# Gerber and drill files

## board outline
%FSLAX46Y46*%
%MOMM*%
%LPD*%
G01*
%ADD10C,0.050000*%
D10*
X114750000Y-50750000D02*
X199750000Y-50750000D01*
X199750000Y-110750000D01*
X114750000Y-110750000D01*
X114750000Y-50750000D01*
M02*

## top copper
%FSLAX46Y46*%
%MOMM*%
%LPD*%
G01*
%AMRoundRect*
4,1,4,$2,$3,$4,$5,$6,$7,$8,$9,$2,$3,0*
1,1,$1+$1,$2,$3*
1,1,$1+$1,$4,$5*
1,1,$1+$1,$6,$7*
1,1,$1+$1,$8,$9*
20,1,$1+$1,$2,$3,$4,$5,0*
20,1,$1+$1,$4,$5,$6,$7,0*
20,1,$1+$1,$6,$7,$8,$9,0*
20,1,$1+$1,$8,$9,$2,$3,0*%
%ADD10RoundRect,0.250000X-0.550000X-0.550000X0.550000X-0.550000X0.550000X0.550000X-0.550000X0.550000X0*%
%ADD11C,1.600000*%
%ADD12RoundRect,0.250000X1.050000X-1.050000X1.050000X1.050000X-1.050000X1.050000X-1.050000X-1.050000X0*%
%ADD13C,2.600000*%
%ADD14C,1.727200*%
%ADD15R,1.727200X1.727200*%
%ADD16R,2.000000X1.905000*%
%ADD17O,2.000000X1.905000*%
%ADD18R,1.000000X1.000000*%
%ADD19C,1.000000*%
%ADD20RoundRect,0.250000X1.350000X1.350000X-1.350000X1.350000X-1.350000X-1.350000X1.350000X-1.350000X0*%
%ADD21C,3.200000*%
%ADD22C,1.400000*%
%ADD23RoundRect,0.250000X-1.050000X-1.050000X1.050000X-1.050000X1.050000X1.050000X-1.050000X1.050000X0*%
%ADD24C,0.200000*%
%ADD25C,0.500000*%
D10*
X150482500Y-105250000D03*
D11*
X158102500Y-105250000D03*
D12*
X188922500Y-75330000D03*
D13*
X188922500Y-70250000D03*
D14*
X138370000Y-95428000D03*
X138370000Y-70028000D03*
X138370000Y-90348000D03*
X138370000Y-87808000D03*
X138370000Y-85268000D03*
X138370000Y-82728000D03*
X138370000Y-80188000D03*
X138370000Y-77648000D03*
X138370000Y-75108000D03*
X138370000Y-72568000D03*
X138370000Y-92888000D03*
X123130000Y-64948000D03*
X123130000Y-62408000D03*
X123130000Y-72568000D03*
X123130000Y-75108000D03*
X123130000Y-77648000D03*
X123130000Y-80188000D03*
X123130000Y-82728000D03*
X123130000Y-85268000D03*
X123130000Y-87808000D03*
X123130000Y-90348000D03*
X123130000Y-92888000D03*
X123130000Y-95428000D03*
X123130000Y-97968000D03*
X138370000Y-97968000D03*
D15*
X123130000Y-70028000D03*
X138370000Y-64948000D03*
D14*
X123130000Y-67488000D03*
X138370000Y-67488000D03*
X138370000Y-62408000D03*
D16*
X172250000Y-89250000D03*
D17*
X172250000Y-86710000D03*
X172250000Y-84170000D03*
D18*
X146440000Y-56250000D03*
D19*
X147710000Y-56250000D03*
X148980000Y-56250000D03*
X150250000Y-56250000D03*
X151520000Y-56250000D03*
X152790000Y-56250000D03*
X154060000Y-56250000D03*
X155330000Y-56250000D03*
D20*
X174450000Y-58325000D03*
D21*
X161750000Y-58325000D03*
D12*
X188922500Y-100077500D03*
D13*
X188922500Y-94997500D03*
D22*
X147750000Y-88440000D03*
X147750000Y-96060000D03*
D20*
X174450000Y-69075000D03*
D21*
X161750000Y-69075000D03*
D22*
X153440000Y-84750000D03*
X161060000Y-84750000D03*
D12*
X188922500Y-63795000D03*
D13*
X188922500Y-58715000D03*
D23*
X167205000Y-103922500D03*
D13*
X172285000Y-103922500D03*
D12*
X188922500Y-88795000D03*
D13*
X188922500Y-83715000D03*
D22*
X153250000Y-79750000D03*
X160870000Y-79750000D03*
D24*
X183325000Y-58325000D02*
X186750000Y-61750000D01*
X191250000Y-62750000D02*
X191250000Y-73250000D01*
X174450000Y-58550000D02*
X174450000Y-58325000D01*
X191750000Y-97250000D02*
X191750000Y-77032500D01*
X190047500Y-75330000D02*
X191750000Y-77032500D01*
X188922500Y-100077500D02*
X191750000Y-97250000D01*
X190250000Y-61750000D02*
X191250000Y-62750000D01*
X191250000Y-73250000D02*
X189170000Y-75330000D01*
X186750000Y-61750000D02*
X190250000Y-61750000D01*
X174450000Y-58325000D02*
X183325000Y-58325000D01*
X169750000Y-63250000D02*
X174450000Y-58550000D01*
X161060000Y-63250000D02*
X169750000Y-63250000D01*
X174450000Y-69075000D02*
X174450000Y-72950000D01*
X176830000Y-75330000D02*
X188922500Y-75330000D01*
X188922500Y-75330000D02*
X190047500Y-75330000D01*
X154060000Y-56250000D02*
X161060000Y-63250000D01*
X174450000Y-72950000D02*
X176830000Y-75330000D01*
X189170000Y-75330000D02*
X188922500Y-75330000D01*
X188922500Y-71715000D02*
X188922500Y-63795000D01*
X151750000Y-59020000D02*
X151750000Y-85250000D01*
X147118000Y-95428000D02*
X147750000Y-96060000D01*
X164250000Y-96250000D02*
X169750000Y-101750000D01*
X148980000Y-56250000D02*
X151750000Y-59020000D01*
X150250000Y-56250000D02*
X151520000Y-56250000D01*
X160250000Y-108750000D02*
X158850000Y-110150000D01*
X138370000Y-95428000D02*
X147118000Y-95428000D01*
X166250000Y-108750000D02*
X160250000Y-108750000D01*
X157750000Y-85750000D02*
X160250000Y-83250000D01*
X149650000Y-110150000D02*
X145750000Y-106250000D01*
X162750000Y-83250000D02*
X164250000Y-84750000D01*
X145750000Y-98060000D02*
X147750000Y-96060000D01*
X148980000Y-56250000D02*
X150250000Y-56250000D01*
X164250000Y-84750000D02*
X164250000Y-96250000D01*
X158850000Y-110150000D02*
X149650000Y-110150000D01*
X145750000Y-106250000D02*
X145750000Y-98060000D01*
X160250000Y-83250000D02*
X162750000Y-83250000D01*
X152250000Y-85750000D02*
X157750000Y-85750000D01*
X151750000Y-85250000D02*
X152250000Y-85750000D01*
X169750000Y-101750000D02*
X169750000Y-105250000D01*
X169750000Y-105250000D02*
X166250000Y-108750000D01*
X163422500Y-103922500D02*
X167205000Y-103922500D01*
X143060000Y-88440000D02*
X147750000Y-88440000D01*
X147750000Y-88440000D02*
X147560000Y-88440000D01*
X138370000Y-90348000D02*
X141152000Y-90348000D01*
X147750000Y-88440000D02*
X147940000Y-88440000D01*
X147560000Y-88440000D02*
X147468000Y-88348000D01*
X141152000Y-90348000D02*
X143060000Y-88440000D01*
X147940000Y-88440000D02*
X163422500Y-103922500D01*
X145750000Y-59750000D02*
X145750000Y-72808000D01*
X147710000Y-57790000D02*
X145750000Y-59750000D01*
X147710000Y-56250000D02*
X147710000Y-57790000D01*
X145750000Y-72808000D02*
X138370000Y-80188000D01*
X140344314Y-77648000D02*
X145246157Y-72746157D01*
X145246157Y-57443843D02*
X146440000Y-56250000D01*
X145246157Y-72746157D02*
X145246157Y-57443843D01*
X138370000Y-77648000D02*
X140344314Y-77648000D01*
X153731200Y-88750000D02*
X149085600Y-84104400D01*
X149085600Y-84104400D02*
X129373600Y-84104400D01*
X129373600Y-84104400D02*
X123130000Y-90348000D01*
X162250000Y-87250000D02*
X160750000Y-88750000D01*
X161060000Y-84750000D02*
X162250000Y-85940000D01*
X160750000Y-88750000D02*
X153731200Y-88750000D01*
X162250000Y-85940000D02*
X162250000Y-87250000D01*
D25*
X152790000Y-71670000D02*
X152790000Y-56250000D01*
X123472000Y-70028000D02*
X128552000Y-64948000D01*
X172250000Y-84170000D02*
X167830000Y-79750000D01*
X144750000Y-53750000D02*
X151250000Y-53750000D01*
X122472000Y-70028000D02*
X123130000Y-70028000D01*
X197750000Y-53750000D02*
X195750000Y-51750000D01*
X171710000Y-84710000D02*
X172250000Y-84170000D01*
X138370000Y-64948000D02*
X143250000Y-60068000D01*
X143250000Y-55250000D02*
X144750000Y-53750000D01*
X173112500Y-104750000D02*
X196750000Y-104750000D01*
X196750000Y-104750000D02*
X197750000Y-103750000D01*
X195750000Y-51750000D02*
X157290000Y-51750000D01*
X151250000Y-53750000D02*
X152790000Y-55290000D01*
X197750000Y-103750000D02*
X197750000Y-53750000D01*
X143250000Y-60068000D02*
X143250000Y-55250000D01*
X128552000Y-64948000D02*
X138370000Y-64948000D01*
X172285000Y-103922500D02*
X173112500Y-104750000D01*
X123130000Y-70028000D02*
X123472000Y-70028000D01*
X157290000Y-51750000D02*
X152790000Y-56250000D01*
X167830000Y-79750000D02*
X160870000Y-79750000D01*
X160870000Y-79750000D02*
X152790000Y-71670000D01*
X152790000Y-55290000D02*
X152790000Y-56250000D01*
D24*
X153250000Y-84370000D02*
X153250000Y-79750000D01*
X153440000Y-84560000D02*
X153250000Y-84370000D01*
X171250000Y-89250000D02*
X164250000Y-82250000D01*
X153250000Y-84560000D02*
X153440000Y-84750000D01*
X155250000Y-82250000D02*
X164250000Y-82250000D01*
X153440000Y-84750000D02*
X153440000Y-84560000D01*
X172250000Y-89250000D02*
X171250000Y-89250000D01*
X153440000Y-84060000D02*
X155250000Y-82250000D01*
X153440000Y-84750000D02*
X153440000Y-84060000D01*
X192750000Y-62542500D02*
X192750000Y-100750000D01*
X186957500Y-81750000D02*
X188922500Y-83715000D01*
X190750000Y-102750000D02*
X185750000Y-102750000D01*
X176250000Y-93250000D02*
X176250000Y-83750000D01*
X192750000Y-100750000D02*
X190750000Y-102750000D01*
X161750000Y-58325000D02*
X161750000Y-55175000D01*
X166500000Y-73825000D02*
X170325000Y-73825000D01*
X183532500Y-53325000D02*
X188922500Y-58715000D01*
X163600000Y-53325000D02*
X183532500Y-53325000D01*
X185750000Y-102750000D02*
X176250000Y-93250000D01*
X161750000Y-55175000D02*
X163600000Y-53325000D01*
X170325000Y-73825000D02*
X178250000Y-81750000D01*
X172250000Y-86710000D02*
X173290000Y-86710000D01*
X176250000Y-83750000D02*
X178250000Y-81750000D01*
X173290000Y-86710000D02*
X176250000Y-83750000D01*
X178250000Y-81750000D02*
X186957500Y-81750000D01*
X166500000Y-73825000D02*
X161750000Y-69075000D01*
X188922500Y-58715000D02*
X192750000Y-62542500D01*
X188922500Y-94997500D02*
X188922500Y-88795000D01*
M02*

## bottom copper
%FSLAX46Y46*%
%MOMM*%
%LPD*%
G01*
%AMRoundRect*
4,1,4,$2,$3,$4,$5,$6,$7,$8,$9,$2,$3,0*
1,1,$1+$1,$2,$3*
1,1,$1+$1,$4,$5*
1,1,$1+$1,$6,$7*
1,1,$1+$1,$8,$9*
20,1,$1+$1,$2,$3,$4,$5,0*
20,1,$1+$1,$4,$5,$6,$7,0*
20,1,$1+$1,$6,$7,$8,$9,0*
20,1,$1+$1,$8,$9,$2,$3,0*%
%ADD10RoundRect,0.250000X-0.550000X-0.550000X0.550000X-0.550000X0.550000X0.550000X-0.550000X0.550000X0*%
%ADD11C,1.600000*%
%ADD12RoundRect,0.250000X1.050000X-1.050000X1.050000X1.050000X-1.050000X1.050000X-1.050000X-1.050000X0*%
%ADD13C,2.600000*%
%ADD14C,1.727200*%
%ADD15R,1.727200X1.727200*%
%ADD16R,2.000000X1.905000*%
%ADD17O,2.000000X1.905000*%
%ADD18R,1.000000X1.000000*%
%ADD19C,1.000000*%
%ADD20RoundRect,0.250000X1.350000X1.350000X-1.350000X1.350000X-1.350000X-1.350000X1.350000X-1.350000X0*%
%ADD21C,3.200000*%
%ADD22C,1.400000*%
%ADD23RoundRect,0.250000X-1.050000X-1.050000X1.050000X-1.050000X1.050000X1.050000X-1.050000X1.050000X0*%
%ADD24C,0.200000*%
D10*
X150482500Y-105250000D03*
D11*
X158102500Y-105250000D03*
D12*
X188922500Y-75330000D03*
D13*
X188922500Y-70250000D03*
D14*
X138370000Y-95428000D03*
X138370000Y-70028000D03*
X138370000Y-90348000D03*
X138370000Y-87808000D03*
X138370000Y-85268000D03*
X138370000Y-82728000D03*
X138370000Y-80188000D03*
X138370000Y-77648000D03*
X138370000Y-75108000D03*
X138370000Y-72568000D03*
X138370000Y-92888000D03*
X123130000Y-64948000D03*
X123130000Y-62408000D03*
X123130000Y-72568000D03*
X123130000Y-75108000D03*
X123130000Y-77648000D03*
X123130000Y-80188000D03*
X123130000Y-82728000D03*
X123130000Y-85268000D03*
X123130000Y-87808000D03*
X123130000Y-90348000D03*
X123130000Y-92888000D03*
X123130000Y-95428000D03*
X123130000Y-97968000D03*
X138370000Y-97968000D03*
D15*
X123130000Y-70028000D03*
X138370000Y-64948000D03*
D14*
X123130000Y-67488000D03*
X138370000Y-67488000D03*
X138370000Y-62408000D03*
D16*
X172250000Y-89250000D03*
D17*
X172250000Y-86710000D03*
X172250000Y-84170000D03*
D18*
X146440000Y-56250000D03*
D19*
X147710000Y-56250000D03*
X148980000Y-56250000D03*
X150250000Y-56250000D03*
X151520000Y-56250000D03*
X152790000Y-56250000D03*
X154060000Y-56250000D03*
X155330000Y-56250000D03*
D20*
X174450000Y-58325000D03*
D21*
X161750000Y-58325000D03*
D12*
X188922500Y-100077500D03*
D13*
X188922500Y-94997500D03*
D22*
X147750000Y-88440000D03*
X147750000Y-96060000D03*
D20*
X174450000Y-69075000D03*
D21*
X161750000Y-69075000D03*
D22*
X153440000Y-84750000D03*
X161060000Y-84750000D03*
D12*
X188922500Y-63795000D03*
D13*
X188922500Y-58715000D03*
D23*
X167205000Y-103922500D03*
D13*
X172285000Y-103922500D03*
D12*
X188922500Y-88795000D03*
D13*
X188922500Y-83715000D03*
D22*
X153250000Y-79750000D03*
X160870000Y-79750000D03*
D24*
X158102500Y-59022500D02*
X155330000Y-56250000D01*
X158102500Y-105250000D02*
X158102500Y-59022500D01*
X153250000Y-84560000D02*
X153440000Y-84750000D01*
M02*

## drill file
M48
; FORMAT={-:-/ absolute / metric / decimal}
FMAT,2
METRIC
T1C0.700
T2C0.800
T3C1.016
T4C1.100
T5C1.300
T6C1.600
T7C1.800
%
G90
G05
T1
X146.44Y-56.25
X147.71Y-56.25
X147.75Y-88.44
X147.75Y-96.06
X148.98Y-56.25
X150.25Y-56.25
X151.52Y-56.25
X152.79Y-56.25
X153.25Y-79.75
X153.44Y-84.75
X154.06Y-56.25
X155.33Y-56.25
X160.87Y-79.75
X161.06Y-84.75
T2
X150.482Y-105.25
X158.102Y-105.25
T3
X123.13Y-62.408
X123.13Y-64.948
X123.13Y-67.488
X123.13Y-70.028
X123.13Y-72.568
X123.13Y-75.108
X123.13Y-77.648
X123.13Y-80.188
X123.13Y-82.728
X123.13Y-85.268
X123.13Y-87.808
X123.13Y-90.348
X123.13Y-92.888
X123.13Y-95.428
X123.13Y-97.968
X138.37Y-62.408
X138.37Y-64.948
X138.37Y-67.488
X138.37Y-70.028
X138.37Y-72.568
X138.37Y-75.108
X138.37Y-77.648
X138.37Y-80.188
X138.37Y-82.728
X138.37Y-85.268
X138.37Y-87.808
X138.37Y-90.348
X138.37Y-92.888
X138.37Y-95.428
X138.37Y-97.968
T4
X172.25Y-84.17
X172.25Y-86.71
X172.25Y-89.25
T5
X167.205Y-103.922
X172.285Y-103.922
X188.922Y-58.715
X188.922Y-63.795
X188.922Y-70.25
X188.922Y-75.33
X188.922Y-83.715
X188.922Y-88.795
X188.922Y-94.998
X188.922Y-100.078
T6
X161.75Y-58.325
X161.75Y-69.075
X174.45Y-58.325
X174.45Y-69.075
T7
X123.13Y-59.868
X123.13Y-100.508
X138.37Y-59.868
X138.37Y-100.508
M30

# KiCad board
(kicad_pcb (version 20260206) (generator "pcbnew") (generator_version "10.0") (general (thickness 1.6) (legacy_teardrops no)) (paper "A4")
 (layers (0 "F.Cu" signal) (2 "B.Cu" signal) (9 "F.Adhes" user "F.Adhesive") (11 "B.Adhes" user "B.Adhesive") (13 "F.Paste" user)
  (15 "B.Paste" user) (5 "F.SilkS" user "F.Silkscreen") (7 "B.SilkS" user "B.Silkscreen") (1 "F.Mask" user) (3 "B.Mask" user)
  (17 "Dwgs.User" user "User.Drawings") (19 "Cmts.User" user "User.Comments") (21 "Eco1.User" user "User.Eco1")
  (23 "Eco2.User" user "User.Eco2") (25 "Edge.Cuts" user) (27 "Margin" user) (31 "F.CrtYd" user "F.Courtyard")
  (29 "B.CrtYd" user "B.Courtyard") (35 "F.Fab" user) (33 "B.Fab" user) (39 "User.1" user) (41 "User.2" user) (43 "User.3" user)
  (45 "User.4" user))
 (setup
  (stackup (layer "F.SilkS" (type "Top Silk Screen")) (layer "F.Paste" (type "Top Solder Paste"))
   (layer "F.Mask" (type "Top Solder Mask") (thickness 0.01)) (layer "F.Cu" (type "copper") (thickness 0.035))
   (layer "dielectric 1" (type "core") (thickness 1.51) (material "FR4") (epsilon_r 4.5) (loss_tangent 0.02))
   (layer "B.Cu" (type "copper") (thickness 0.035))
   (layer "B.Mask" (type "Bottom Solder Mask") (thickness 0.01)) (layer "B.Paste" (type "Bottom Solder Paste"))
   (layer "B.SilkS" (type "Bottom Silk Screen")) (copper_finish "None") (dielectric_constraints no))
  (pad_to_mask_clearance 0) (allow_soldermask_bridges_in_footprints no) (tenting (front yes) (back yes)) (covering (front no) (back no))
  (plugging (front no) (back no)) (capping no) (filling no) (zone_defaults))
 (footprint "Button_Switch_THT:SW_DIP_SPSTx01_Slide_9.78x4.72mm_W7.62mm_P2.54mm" (layer "F.Cu") (at 150.4825 105.25)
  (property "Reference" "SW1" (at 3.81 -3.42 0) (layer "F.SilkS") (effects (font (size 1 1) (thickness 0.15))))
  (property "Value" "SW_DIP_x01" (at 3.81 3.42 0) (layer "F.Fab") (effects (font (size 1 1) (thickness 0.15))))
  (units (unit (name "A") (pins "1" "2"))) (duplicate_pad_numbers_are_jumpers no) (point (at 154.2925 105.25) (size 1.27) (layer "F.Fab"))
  (pad "1" thru_hole roundrect (at 0 0) (size 1.6 1.6) (drill 0.8) (layers "*.Cu" "*.Mask") (remove_unused_layers no)
   (roundrect_rratio 0.15625) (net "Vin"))
  (pad "2" thru_hole circle (at 7.62 0) (size 1.6 1.6) (drill 0.8) (layers "*.Cu" "*.Mask") (remove_unused_layers no) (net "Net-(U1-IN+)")))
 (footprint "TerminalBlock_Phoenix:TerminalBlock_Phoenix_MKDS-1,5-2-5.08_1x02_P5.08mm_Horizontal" (layer "F.Cu") (at 188.9225 75.33 90)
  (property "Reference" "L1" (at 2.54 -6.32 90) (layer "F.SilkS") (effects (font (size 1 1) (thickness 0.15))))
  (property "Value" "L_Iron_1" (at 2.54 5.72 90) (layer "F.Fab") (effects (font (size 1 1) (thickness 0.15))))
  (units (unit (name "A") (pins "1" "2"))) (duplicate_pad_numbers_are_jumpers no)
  (pad "1" thru_hole roundrect (at 0 0 90) (size 2.6 2.6) (drill 1.3) (layers "*.Cu" "*.Mask") (remove_unused_layers no)
   (roundrect_rratio 0.096154) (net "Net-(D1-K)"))
  (pad "2" thru_hole circle (at 5.08 0 90) (size 2.6 2.6) (drill 1.3) (layers "*.Cu" "*.Mask") (remove_unused_layers no)
   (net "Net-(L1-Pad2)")))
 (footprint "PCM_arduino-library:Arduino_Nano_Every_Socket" (layer "F.Cu") (at 130.75 101.778)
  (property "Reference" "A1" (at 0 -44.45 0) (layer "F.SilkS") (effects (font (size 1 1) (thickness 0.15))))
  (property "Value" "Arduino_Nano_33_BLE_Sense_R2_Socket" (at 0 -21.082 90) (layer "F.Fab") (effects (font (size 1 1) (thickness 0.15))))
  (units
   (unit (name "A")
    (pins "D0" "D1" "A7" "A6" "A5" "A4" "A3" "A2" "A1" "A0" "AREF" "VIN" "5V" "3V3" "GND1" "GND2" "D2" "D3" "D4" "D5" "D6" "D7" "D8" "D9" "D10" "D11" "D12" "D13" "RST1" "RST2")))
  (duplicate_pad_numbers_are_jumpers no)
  (pad "" np_thru_hole circle (at -7.62 -41.91) (size 1.8 1.8) (drill 1.8) (layers "*.Cu" "*.Mask"))
  (pad "" np_thru_hole circle (at -7.62 -1.27) (size 1.8 1.8) (drill 1.8) (layers "*.Cu" "*.Mask"))
  (pad "" np_thru_hole circle (at 7.62 -41.91) (size 1.8 1.8) (drill 1.8) (layers "*.Cu" "*.Mask"))
  (pad "" np_thru_hole circle (at 7.62 -1.27) (size 1.8 1.8) (drill 1.8) (layers "*.Cu" "*.Mask"))
  (pad "3V3" thru_hole circle (at 7.62 -6.35) (size 1.7272 1.7272) (drill 1.016) (layers "*.Cu" "*.Mask") (remove_unused_layers no)
   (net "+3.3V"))
  (pad "5V" thru_hole circle (at 7.62 -31.75) (size 1.7272 1.7272) (drill 1.016) (layers "*.Cu" "*.Mask") (remove_unused_layers no)
   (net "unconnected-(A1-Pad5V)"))
  (pad "A0" thru_hole circle (at 7.62 -11.43) (size 1.7272 1.7272) (drill 1.016) (layers "*.Cu" "*.Mask") (remove_unused_layers no)
   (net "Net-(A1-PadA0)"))
  (pad "A1" thru_hole circle (at 7.62 -13.97) (size 1.7272 1.7272) (drill 1.016) (layers "*.Cu" "*.Mask") (remove_unused_layers no)
   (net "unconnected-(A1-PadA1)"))
  (pad "A2" thru_hole circle (at 7.62 -16.51) (size 1.7272 1.7272) (drill 1.016) (layers "*.Cu" "*.Mask") (remove_unused_layers no)
   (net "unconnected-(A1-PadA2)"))
  (pad "A3" thru_hole circle (at 7.62 -19.05) (size 1.7272 1.7272) (drill 1.016) (layers "*.Cu" "*.Mask") (remove_unused_layers no)
   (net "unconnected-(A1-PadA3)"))
  (pad "A4" thru_hole circle (at 7.62 -21.59) (size 1.7272 1.7272) (drill 1.016) (layers "*.Cu" "*.Mask") (remove_unused_layers no)
   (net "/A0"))
  (pad "A5" thru_hole circle (at 7.62 -24.13) (size 1.7272 1.7272) (drill 1.016) (layers "*.Cu" "*.Mask") (remove_unused_layers no)
   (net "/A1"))
  (pad "A6" thru_hole circle (at 7.62 -26.67) (size 1.7272 1.7272) (drill 1.016) (layers "*.Cu" "*.Mask") (remove_unused_layers no)
   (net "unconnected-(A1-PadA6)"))
  (pad "A7" thru_hole circle (at 7.62 -29.21) (size 1.7272 1.7272) (drill 1.016) (layers "*.Cu" "*.Mask") (remove_unused_layers no)
   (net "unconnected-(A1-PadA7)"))
  (pad "AREF" thru_hole circle (at 7.62 -8.89) (size 1.7272 1.7272) (drill 1.016) (layers "*.Cu" "*.Mask") (remove_unused_layers no)
   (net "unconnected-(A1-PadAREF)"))
  (pad "D0" thru_hole circle (at -7.62 -36.83) (size 1.7272 1.7272) (drill 1.016) (layers "*.Cu" "*.Mask") (remove_unused_layers no)
   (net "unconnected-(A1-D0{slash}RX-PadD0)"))
  (pad "D1" thru_hole circle (at -7.62 -39.37) (size 1.7272 1.7272) (drill 1.016) (layers "*.Cu" "*.Mask") (remove_unused_layers no)
   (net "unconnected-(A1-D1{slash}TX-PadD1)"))
  (pad "D2" thru_hole circle (at -7.62 -29.21) (size 1.7272 1.7272) (drill 1.016) (layers "*.Cu" "*.Mask") (remove_unused_layers no)
   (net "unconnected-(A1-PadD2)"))
  (pad "D3" thru_hole circle (at -7.62 -26.67) (size 1.7272 1.7272) (drill 1.016) (layers "*.Cu" "*.Mask") (remove_unused_layers no)
   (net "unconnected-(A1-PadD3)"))
  (pad "D4" thru_hole circle (at -7.62 -24.13) (size 1.7272 1.7272) (drill 1.016) (layers "*.Cu" "*.Mask") (remove_unused_layers no)
   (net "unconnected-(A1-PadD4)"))
  (pad "D5" thru_hole circle (at -7.62 -21.59) (size 1.7272 1.7272) (drill 1.016) (layers "*.Cu" "*.Mask") (remove_unused_layers no)
   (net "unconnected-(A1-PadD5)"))
  (pad "D6" thru_hole circle (at -7.62 -19.05) (size 1.7272 1.7272) (drill 1.016) (layers "*.Cu" "*.Mask") (remove_unused_layers no)
   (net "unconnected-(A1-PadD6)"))
  (pad "D7" thru_hole circle (at -7.62 -16.51) (size 1.7272 1.7272) (drill 1.016) (layers "*.Cu" "*.Mask") (remove_unused_layers no)
   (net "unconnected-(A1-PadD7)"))
  (pad "D8" thru_hole circle (at -7.62 -13.97) (size 1.7272 1.7272) (drill 1.016) (layers "*.Cu" "*.Mask") (remove_unused_layers no)
   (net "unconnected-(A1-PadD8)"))
  (pad "D9" thru_hole circle (at -7.62 -11.43) (size 1.7272 1.7272) (drill 1.016) (layers "*.Cu" "*.Mask") (remove_unused_layers no)
   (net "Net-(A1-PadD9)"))
  (pad "D10" thru_hole circle (at -7.62 -8.89) (size 1.7272 1.7272) (drill 1.016) (layers "*.Cu" "*.Mask") (remove_unused_layers no)
   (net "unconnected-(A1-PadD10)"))
  (pad "D11" thru_hole circle (at -7.62 -6.35) (size 1.7272 1.7272) (drill 1.016) (layers "*.Cu" "*.Mask") (remove_unused_layers no)
   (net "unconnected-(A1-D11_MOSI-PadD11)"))
  (pad "D12" thru_hole circle (at -7.62 -3.81) (size 1.7272 1.7272) (drill 1.016) (layers "*.Cu" "*.Mask") (remove_unused_layers no)
   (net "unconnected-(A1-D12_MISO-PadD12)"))
  (pad "D13" thru_hole circle (at 7.62 -3.81) (size 1.7272 1.7272) (drill 1.016) (layers "*.Cu" "*.Mask") (remove_unused_layers no)
   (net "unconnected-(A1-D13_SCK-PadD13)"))
  (pad "GND1" thru_hole rect (at -7.62 -31.75) (size 1.7272 1.7272) (drill 1.016) (layers "*.Cu" "*.Mask") (remove_unused_layers no)
   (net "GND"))
  (pad "GND2" thru_hole rect (at 7.62 -36.83) (size 1.7272 1.7272) (drill 1.016) (layers "*.Cu" "*.Mask") (remove_unused_layers no)
   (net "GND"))
  (pad "RST1" thru_hole circle (at -7.62 -34.29) (size 1.7272 1.7272) (drill 1.016) (layers "*.Cu" "*.Mask") (remove_unused_layers no)
   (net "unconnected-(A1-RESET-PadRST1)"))
  (pad "RST2" thru_hole circle (at 7.62 -34.29) (size 1.7272 1.7272) (drill 1.016) (layers "*.Cu" "*.Mask") (remove_unused_layers no)
   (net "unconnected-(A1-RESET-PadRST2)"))
  (pad "VIN" thru_hole circle (at 7.62 -39.37) (size 1.7272 1.7272) (drill 1.016) (layers "*.Cu" "*.Mask") (remove_unused_layers no)
   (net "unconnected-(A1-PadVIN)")))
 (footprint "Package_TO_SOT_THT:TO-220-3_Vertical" (layer "F.Cu") (at 172.25 89.25 90)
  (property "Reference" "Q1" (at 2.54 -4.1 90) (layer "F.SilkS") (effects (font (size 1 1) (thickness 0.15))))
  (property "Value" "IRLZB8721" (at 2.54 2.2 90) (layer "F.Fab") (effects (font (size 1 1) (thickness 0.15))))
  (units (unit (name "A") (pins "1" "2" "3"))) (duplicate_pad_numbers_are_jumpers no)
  (pad "1" thru_hole rect (at 0 0 90) (size 1.905 2) (drill 1.1) (layers "*.Cu" "*.Mask") (remove_unused_layers no) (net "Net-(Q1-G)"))
  (pad "2" thru_hole oval (at 2.54 0 90) (size 1.905 2) (drill 1.1) (layers "*.Cu" "*.Mask") (remove_unused_layers no) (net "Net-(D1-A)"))
  (pad "3" thru_hole oval (at 5.08 0 90) (size 1.905 2) (drill 1.1) (layers "*.Cu" "*.Mask") (remove_unused_layers no) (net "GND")))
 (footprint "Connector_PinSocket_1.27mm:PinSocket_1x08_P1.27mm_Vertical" (layer "F.Cu") (at 146.44 56.25 90)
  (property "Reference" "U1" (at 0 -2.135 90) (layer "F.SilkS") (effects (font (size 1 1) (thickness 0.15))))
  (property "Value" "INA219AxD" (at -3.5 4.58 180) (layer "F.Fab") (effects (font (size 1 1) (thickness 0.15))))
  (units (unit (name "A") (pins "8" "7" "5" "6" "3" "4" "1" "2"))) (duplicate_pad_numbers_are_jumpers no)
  (pad "1" thru_hole rect (at 0 0 90) (size 1 1) (drill 0.7) (layers "*.Cu" "*.Mask") (remove_unused_layers no) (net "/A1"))
  (pad "2" thru_hole circle (at 0 1.27 90) (size 1 1) (drill 0.7) (layers "*.Cu" "*.Mask") (remove_unused_layers no) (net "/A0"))
  (pad "3" thru_hole circle (at 0 2.54 90) (size 1 1) (drill 0.7) (layers "*.Cu" "*.Mask") (remove_unused_layers no) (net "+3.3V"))
  (pad "4" thru_hole circle (at 0 3.81 90) (size 1 1) (drill 0.7) (layers "*.Cu" "*.Mask") (remove_unused_layers no) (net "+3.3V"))
  (pad "5" thru_hole circle (at 0 5.08 90) (size 1 1) (drill 0.7) (layers "*.Cu" "*.Mask") (remove_unused_layers no) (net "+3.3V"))
  (pad "6" thru_hole circle (at 0 6.35 90) (size 1 1) (drill 0.7) (layers "*.Cu" "*.Mask") (remove_unused_layers no) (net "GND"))
  (pad "7" thru_hole circle (at 0 7.62 90) (size 1 1) (drill 0.7) (layers "*.Cu" "*.Mask") (remove_unused_layers no) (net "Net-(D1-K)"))
  (pad "8" thru_hole circle (at 0 8.89 90) (size 1 1) (drill 0.7) (layers "*.Cu" "*.Mask") (remove_unused_layers no) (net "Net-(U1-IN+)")))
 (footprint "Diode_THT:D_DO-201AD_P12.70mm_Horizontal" (layer "F.Cu") (at 174.45 58.325 180)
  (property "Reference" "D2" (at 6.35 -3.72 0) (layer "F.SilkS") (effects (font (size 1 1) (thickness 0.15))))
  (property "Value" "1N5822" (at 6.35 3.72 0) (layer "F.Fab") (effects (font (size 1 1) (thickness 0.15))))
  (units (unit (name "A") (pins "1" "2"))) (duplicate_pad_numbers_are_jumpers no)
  (pad "1" thru_hole roundrect (at 0 0 180) (size 3.2 3.2) (drill 1.6) (layers "*.Cu" "*.Mask") (remove_unused_layers no)
   (roundrect_rratio 0.078125) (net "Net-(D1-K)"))
  (pad "2" thru_hole circle (at 12.7 0 180) (size 3.2 3.2) (drill 1.6) (layers "*.Cu" "*.Mask") (remove_unused_layers no) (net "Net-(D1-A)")))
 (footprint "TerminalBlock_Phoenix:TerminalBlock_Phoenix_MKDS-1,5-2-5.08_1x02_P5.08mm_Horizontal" (layer "F.Cu") (at 188.9225 100.0775 90)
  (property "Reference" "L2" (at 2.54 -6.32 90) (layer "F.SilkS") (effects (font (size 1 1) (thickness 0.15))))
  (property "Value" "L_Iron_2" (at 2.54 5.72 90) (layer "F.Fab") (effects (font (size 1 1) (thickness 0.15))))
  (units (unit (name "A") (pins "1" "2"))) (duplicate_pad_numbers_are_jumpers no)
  (pad "1" thru_hole roundrect (at 0 0 90) (size 2.6 2.6) (drill 1.3) (layers "*.Cu" "*.Mask") (remove_unused_layers no)
   (roundrect_rratio 0.096154) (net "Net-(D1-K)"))
  (pad "2" thru_hole circle (at 5.08 0 90) (size 2.6 2.6) (drill 1.3) (layers "*.Cu" "*.Mask") (remove_unused_layers no)
   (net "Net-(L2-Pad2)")))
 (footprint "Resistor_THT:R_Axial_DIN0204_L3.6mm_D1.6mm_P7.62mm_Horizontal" (layer "F.Cu") (at 147.75 88.44 -90)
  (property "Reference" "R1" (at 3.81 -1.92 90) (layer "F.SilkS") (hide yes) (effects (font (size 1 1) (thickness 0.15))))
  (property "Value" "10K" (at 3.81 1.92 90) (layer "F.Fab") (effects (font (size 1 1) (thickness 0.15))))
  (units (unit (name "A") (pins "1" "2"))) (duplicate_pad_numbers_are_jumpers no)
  (pad "1" thru_hole circle (at 0 0 270) (size 1.4 1.4) (drill 0.7) (layers "*.Cu" "*.Mask") (remove_unused_layers no)
   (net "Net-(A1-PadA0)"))
  (pad "2" thru_hole circle (at 7.62 0 270) (size 1.4 1.4) (drill 0.7) (layers "*.Cu" "*.Mask") (remove_unused_layers no) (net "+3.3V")))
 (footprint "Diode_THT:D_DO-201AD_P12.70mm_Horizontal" (layer "F.Cu") (at 174.45 69.075 180)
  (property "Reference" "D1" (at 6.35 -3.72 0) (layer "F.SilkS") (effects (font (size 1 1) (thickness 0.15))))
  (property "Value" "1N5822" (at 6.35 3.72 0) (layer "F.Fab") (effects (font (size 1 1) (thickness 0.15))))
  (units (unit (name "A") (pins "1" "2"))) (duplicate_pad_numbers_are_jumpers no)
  (pad "1" thru_hole roundrect (at 0 0 180) (size 3.2 3.2) (drill 1.6) (layers "*.Cu" "*.Mask") (remove_unused_layers no)
   (roundrect_rratio 0.078125) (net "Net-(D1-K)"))
  (pad "2" thru_hole circle (at 12.7 0 180) (size 3.2 3.2) (drill 1.6) (layers "*.Cu" "*.Mask") (remove_unused_layers no) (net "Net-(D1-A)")))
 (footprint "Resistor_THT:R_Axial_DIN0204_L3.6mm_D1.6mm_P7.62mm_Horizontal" (layer "F.Cu") (at 153.44 84.75)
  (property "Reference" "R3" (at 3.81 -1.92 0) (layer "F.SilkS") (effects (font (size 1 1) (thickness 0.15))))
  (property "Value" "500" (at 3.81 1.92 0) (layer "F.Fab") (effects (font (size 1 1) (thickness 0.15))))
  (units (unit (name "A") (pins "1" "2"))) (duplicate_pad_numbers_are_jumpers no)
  (pad "1" thru_hole circle (at 0 0) (size 1.4 1.4) (drill 0.7) (layers "*.Cu" "*.Mask") (remove_unused_layers no) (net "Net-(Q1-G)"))
  (pad "2" thru_hole circle (at 7.62 0) (size 1.4 1.4) (drill 0.7) (layers "*.Cu" "*.Mask") (remove_unused_layers no) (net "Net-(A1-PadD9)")))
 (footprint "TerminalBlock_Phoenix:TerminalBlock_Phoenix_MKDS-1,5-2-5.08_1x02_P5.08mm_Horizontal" (layer "F.Cu") (at 188.9225 63.795 90)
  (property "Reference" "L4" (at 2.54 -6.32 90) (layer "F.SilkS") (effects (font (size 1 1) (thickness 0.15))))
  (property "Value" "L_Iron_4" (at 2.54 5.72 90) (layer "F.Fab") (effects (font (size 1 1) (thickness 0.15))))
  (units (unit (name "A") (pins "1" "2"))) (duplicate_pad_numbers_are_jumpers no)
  (pad "1" thru_hole roundrect (at 0 0 90) (size 2.6 2.6) (drill 1.3) (layers "*.Cu" "*.Mask") (remove_unused_layers no)
   (roundrect_rratio 0.096154) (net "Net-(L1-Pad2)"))
  (pad "2" thru_hole circle (at 5.08 0 90) (size 2.6 2.6) (drill 1.3) (layers "*.Cu" "*.Mask") (remove_unused_layers no) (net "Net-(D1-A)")))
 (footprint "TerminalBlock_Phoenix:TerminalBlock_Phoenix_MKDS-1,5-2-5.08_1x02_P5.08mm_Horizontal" (layer "F.Cu") (at 167.205 103.9225)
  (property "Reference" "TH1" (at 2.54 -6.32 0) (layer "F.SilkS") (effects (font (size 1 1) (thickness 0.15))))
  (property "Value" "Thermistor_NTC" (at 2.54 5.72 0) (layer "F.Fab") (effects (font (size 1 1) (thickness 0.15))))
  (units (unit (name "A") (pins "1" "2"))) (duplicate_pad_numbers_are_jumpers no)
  (pad "1" thru_hole roundrect (at 0 0) (size 2.6 2.6) (drill 1.3) (layers "*.Cu" "*.Mask") (remove_unused_layers no)
   (roundrect_rratio 0.096154) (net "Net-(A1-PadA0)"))
  (pad "2" thru_hole circle (at 5.08 0) (size 2.6 2.6) (drill 1.3) (layers "*.Cu" "*.Mask") (remove_unused_layers no) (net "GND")))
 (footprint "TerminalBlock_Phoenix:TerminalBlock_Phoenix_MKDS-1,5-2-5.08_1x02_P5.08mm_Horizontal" (layer "F.Cu") (at 188.9225 88.795 90)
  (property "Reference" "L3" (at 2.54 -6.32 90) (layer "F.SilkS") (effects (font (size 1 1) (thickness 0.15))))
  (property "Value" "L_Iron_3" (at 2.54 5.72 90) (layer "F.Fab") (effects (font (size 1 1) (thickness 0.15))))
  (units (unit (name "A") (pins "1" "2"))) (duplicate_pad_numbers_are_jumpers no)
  (pad "1" thru_hole roundrect (at 0 0 90) (size 2.6 2.6) (drill 1.3) (layers "*.Cu" "*.Mask") (remove_unused_layers no)
   (roundrect_rratio 0.096154) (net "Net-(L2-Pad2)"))
  (pad "2" thru_hole circle (at 5.08 0 90) (size 2.6 2.6) (drill 1.3) (layers "*.Cu" "*.Mask") (remove_unused_layers no) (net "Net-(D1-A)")))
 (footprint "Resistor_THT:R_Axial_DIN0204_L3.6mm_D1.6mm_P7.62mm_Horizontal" (layer "F.Cu") (at 153.25 79.75)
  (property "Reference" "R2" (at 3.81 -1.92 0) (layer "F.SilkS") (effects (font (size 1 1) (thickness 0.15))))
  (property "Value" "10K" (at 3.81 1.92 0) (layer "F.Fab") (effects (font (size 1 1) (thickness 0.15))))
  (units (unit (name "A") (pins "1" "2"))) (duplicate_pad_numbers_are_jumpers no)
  (pad "1" thru_hole circle (at 0 0) (size 1.4 1.4) (drill 0.7) (layers "*.Cu" "*.Mask") (remove_unused_layers no) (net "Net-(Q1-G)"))
  (pad "2" thru_hole circle (at 7.62 0) (size 1.4 1.4) (drill 0.7) (layers "*.Cu" "*.Mask") (remove_unused_layers no) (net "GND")))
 (gr_rect (start 114.75 50.75) (end 199.75 110.75) (stroke (width 0.05) (type default)) (fill no) (layer "Edge.Cuts"))
 (segment (start 158.1025 59.0225) (end 155.33 56.25) (width 0.2) (layer "B.Cu") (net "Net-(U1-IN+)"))
 (segment (start 158.1025 105.25) (end 158.1025 59.0225) (width 0.2) (layer "B.Cu") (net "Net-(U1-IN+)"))
 (segment (start 183.325 58.325) (end 186.75 61.75) (width 0.2) (layer "F.Cu") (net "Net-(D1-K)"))
 (segment (start 191.25 62.75) (end 191.25 73.25) (width 0.2) (layer "F.Cu") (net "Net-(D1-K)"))
 (segment (start 174.45 58.55) (end 174.45 58.325) (width 0.2) (layer "F.Cu") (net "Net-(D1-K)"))
 (segment (start 191.75 97.25) (end 191.75 77.0325) (width 0.2) (layer "F.Cu") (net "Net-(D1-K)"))
 (segment (start 190.0475 75.33) (end 191.75 77.0325) (width 0.2) (layer "F.Cu") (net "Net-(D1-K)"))
 (segment (start 188.9225 100.0775) (end 191.75 97.25) (width 0.2) (layer "F.Cu") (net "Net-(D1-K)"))
 (segment (start 190.25 61.75) (end 191.25 62.75) (width 0.2) (layer "F.Cu") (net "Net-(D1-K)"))
 (segment (start 191.25 73.25) (end 189.17 75.33) (width 0.2) (layer "F.Cu") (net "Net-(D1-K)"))
 (segment (start 186.75 61.75) (end 190.25 61.75) (width 0.2) (layer "F.Cu") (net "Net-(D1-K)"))
 (segment (start 174.45 58.325) (end 183.325 58.325) (width 0.2) (layer "F.Cu") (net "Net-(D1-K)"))
 (segment (start 169.75 63.25) (end 174.45 58.55) (width 0.2) (layer "F.Cu") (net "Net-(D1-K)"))
 (segment (start 161.06 63.25) (end 169.75 63.25) (width 0.2) (layer "F.Cu") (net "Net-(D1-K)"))
 (segment (start 174.45 69.075) (end 174.45 72.95) (width 0.2) (layer "F.Cu") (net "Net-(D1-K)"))
 (segment (start 176.83 75.33) (end 188.9225 75.33) (width 0.2) (layer "F.Cu") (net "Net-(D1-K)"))
 (segment (start 188.9225 75.33) (end 190.0475 75.33) (width 0.2) (layer "F.Cu") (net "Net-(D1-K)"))
 (segment (start 154.06 56.25) (end 161.06 63.25) (width 0.2) (layer "F.Cu") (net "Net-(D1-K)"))
 (segment (start 174.45 72.95) (end 176.83 75.33) (width 0.2) (layer "F.Cu") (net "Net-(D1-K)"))
 (segment (start 189.17 75.33) (end 188.9225 75.33) (width 0.2) (layer "F.Cu") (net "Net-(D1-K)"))
 (segment (start 188.9225 71.715) (end 188.9225 63.795) (width 0.2) (layer "F.Cu") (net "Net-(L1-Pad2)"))
 (segment (start 151.75 59.02) (end 151.75 85.25) (width 0.2) (layer "F.Cu") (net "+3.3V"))
 (segment (start 147.118 95.428) (end 147.75 96.06) (width 0.2) (layer "F.Cu") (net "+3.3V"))
 (segment (start 164.25 96.25) (end 169.75 101.75) (width 0.2) (layer "F.Cu") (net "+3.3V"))
 (segment (start 148.98 56.25) (end 151.75 59.02) (width 0.2) (layer "F.Cu") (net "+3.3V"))
 (segment (start 150.25 56.25) (end 151.52 56.25) (width 0.2) (layer "F.Cu") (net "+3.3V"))
 (segment (start 160.25 108.75) (end 158.85 110.15) (width 0.2) (layer "F.Cu") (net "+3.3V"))
 (segment (start 138.37 95.428) (end 147.118 95.428) (width 0.2) (layer "F.Cu") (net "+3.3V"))
 (segment (start 166.25 108.75) (end 160.25 108.75) (width 0.2) (layer "F.Cu") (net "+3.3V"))
 (segment (start 157.75 85.75) (end 160.25 83.25) (width 0.2) (layer "F.Cu") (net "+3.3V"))
 (segment (start 149.65 110.15) (end 145.75 106.25) (width 0.2) (layer "F.Cu") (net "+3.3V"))
 (segment (start 162.75 83.25) (end 164.25 84.75) (width 0.2) (layer "F.Cu") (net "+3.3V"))
 (segment (start 145.75 98.06) (end 147.75 96.06) (width 0.2) (layer "F.Cu") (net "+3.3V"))
 (segment (start 148.98 56.25) (end 150.25 56.25) (width 0.2) (layer "F.Cu") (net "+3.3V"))
 (segment (start 164.25 84.75) (end 164.25 96.25) (width 0.2) (layer "F.Cu") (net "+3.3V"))
 (segment (start 158.85 110.15) (end 149.65 110.15) (width 0.2) (layer "F.Cu") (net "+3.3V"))
 (segment (start 145.75 106.25) (end 145.75 98.06) (width 0.2) (layer "F.Cu") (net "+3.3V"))
 (segment (start 160.25 83.25) (end 162.75 83.25) (width 0.2) (layer "F.Cu") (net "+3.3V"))
 (segment (start 152.25 85.75) (end 157.75 85.75) (width 0.2) (layer "F.Cu") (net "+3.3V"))
 (segment (start 151.75 85.25) (end 152.25 85.75) (width 0.2) (layer "F.Cu") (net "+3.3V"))
 (segment (start 169.75 101.75) (end 169.75 105.25) (width 0.2) (layer "F.Cu") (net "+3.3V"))
 (segment (start 169.75 105.25) (end 166.25 108.75) (width 0.2) (layer "F.Cu") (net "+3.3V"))
 (segment (start 163.4225 103.9225) (end 167.205 103.9225) (width 0.2) (layer "F.Cu") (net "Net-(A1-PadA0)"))
 (segment (start 143.06 88.44) (end 147.75 88.44) (width 0.2) (layer "F.Cu") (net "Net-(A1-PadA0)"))
 (segment (start 147.75 88.44) (end 147.56 88.44) (width 0.2) (layer "F.Cu") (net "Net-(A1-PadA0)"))
 (segment (start 138.37 90.348) (end 141.152 90.348) (width 0.2) (layer "F.Cu") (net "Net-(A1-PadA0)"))
 (segment (start 147.75 88.44) (end 147.94 88.44) (width 0.2) (layer "F.Cu") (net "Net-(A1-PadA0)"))
 (segment (start 147.56 88.44) (end 147.468 88.348) (width 0.2) (layer "F.Cu") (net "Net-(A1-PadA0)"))
 (segment (start 141.152 90.348) (end 143.06 88.44) (width 0.2) (layer "F.Cu") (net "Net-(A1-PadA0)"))
 (segment (start 147.94 88.44) (end 163.4225 103.9225) (width 0.2) (layer "F.Cu") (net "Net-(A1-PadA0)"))
 (segment (start 145.75 59.75) (end 145.75 72.808) (width 0.2) (layer "F.Cu") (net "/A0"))
 (segment (start 147.71 57.79) (end 145.75 59.75) (width 0.2) (layer "F.Cu") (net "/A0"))
 (segment (start 147.71 56.25) (end 147.71 57.79) (width 0.2) (layer "F.Cu") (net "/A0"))
 (segment (start 145.75 72.808) (end 138.37 80.188) (width 0.2) (layer "F.Cu") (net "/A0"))
 (segment (start 140.344314 77.648) (end 145.246157 72.746157) (width 0.2) (layer "F.Cu") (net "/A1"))
 (segment (start 145.246157 57.443843) (end 146.44 56.25) (width 0.2) (layer "F.Cu") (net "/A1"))
 (segment (start 145.246157 72.746157) (end 145.246157 57.443843) (width 0.2) (layer "F.Cu") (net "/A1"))
 (segment (start 138.37 77.648) (end 140.344314 77.648) (width 0.2) (layer "F.Cu") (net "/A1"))
 (segment (start 153.7312 88.75) (end 149.0856 84.1044) (width 0.2) (layer "F.Cu") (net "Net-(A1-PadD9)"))
 (segment (start 149.0856 84.1044) (end 129.3736 84.1044) (width 0.2) (layer "F.Cu") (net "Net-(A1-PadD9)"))
 (segment (start 129.3736 84.1044) (end 123.13 90.348) (width 0.2) (layer "F.Cu") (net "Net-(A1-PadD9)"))
 (segment (start 162.25 87.25) (end 160.75 88.75) (width 0.2) (layer "F.Cu") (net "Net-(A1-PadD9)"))
 (segment (start 161.06 84.75) (end 162.25 85.94) (width 0.2) (layer "F.Cu") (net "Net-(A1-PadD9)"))
 (segment (start 160.75 88.75) (end 153.7312 88.75) (width 0.2) (layer "F.Cu") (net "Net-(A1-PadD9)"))
 (segment (start 162.25 85.94) (end 162.25 87.25) (width 0.2) (layer "F.Cu") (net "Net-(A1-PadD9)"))
 (segment (start 152.79 71.67) (end 152.79 56.25) (width 0.5) (layer "F.Cu") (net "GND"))
 (segment (start 123.472 70.028) (end 128.552 64.948) (width 0.5) (layer "F.Cu") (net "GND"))
 (segment (start 172.25 84.17) (end 167.83 79.75) (width 0.5) (layer "F.Cu") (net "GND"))
 (segment (start 144.75 53.75) (end 151.25 53.75) (width 0.5) (layer "F.Cu") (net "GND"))
 (segment (start 122.472 70.028) (end 123.13 70.028) (width 0.5) (layer "F.Cu") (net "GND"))
 (segment (start 197.75 53.75) (end 195.75 51.75) (width 0.5) (layer "F.Cu") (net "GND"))
 (segment (start 171.71 84.71) (end 172.25 84.17) (width 0.5) (layer "F.Cu") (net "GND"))
 (segment (start 138.37 64.948) (end 143.25 60.068) (width 0.5) (layer "F.Cu") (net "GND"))
 (segment (start 143.25 55.25) (end 144.75 53.75) (width 0.5) (layer "F.Cu") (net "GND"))
 (segment (start 173.1125 104.75) (end 196.75 104.75) (width 0.5) (layer "F.Cu") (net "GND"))
 (segment (start 196.75 104.75) (end 197.75 103.75) (width 0.5) (layer "F.Cu") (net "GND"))
 (segment (start 195.75 51.75) (end 157.29 51.75) (width 0.5) (layer "F.Cu") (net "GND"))
 (segment (start 151.25 53.75) (end 152.79 55.29) (width 0.5) (layer "F.Cu") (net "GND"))
 (segment (start 197.75 103.75) (end 197.75 53.75) (width 0.5) (layer "F.Cu") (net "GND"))
 (segment (start 143.25 60.068) (end 143.25 55.25) (width 0.5) (layer "F.Cu") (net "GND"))
 (segment (start 128.552 64.948) (end 138.37 64.948) (width 0.5) (layer "F.Cu") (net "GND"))
 (segment (start 172.285 103.9225) (end 173.1125 104.75) (width 0.5) (layer "F.Cu") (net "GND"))
 (segment (start 123.13 70.028) (end 123.472 70.028) (width 0.5) (layer "F.Cu") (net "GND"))
 (segment (start 157.29 51.75) (end 152.79 56.25) (width 0.5) (layer "F.Cu") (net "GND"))
 (segment (start 167.83 79.75) (end 160.87 79.75) (width 0.5) (layer "F.Cu") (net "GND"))
 (segment (start 160.87 79.75) (end 152.79 71.67) (width 0.5) (layer "F.Cu") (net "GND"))
 (segment (start 152.79 55.29) (end 152.79 56.25) (width 0.5) (layer "F.Cu") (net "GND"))
 (segment (start 153.25 84.37) (end 153.25 79.75) (width 0.2) (layer "F.Cu") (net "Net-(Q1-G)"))
 (segment (start 153.44 84.56) (end 153.25 84.37) (width 0.2) (layer "F.Cu") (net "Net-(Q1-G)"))
 (segment (start 171.25 89.25) (end 164.25 82.25) (width 0.2) (layer "F.Cu") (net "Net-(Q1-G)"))
 (segment (start 153.25 84.56) (end 153.44 84.75) (width 0.2) (layer "F.Cu") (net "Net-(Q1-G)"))
 (segment (start 155.25 82.25) (end 164.25 82.25) (width 0.2) (layer "F.Cu") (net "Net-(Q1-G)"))
 (segment (start 153.44 84.75) (end 153.44 84.56) (width 0.2) (layer "F.Cu") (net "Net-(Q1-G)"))
 (segment (start 172.25 89.25) (end 171.25 89.25) (width 0.2) (layer "F.Cu") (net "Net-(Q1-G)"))
 (segment (start 153.44 84.06) (end 155.25 82.25) (width 0.2) (layer "F.Cu") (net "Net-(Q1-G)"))
 (segment (start 153.44 84.75) (end 153.44 84.06) (width 0.2) (layer "F.Cu") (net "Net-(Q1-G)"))
 (segment (start 153.25 84.56) (end 153.44 84.75) (width 0.2) (layer "B.Cu") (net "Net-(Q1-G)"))
 (segment (start 192.75 62.5425) (end 192.75 100.75) (width 0.2) (layer "F.Cu") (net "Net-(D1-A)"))
 (segment (start 186.9575 81.75) (end 188.9225 83.715) (width 0.2) (layer "F.Cu") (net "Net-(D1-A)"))
 (segment (start 190.75 102.75) (end 185.75 102.75) (width 0.2) (layer "F.Cu") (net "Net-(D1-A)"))
 (segment (start 176.25 93.25) (end 176.25 83.75) (width 0.2) (layer "F.Cu") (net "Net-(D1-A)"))
 (segment (start 192.75 100.75) (end 190.75 102.75) (width 0.2) (layer "F.Cu") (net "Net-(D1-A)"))
 (segment (start 161.75 58.325) (end 161.75 55.175) (width 0.2) (layer "F.Cu") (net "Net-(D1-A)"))
 (segment (start 166.5 73.825) (end 170.325 73.825) (width 0.2) (layer "F.Cu") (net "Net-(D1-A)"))
 (segment (start 183.5325 53.325) (end 188.9225 58.715) (width 0.2) (layer "F.Cu") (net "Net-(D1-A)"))
 (segment (start 163.6 53.325) (end 183.5325 53.325) (width 0.2) (layer "F.Cu") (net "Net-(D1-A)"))
 (segment (start 185.75 102.75) (end 176.25 93.25) (width 0.2) (layer "F.Cu") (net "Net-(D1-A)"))
 (segment (start 161.75 55.175) (end 163.6 53.325) (width 0.2) (layer "F.Cu") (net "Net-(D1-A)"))
 (segment (start 170.325 73.825) (end 178.25 81.75) (width 0.2) (layer "F.Cu") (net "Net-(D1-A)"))
 (segment (start 172.25 86.71) (end 173.29 86.71) (width 0.2) (layer "F.Cu") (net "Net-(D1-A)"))
 (segment (start 176.25 83.75) (end 178.25 81.75) (width 0.2) (layer "F.Cu") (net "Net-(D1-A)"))
 (segment (start 173.29 86.71) (end 176.25 83.75) (width 0.2) (layer "F.Cu") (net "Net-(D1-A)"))
 (segment (start 178.25 81.75) (end 186.9575 81.75) (width 0.2) (layer "F.Cu") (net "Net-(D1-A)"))
 (segment (start 166.5 73.825) (end 161.75 69.075) (width 0.2) (layer "F.Cu") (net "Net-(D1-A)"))
 (segment (start 188.9225 58.715) (end 192.75 62.5425) (width 0.2) (layer "F.Cu") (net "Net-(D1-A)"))
 (segment (start 188.9225 94.9975) (end 188.9225 88.795) (width 0.2) (layer "F.Cu") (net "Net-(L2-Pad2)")))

